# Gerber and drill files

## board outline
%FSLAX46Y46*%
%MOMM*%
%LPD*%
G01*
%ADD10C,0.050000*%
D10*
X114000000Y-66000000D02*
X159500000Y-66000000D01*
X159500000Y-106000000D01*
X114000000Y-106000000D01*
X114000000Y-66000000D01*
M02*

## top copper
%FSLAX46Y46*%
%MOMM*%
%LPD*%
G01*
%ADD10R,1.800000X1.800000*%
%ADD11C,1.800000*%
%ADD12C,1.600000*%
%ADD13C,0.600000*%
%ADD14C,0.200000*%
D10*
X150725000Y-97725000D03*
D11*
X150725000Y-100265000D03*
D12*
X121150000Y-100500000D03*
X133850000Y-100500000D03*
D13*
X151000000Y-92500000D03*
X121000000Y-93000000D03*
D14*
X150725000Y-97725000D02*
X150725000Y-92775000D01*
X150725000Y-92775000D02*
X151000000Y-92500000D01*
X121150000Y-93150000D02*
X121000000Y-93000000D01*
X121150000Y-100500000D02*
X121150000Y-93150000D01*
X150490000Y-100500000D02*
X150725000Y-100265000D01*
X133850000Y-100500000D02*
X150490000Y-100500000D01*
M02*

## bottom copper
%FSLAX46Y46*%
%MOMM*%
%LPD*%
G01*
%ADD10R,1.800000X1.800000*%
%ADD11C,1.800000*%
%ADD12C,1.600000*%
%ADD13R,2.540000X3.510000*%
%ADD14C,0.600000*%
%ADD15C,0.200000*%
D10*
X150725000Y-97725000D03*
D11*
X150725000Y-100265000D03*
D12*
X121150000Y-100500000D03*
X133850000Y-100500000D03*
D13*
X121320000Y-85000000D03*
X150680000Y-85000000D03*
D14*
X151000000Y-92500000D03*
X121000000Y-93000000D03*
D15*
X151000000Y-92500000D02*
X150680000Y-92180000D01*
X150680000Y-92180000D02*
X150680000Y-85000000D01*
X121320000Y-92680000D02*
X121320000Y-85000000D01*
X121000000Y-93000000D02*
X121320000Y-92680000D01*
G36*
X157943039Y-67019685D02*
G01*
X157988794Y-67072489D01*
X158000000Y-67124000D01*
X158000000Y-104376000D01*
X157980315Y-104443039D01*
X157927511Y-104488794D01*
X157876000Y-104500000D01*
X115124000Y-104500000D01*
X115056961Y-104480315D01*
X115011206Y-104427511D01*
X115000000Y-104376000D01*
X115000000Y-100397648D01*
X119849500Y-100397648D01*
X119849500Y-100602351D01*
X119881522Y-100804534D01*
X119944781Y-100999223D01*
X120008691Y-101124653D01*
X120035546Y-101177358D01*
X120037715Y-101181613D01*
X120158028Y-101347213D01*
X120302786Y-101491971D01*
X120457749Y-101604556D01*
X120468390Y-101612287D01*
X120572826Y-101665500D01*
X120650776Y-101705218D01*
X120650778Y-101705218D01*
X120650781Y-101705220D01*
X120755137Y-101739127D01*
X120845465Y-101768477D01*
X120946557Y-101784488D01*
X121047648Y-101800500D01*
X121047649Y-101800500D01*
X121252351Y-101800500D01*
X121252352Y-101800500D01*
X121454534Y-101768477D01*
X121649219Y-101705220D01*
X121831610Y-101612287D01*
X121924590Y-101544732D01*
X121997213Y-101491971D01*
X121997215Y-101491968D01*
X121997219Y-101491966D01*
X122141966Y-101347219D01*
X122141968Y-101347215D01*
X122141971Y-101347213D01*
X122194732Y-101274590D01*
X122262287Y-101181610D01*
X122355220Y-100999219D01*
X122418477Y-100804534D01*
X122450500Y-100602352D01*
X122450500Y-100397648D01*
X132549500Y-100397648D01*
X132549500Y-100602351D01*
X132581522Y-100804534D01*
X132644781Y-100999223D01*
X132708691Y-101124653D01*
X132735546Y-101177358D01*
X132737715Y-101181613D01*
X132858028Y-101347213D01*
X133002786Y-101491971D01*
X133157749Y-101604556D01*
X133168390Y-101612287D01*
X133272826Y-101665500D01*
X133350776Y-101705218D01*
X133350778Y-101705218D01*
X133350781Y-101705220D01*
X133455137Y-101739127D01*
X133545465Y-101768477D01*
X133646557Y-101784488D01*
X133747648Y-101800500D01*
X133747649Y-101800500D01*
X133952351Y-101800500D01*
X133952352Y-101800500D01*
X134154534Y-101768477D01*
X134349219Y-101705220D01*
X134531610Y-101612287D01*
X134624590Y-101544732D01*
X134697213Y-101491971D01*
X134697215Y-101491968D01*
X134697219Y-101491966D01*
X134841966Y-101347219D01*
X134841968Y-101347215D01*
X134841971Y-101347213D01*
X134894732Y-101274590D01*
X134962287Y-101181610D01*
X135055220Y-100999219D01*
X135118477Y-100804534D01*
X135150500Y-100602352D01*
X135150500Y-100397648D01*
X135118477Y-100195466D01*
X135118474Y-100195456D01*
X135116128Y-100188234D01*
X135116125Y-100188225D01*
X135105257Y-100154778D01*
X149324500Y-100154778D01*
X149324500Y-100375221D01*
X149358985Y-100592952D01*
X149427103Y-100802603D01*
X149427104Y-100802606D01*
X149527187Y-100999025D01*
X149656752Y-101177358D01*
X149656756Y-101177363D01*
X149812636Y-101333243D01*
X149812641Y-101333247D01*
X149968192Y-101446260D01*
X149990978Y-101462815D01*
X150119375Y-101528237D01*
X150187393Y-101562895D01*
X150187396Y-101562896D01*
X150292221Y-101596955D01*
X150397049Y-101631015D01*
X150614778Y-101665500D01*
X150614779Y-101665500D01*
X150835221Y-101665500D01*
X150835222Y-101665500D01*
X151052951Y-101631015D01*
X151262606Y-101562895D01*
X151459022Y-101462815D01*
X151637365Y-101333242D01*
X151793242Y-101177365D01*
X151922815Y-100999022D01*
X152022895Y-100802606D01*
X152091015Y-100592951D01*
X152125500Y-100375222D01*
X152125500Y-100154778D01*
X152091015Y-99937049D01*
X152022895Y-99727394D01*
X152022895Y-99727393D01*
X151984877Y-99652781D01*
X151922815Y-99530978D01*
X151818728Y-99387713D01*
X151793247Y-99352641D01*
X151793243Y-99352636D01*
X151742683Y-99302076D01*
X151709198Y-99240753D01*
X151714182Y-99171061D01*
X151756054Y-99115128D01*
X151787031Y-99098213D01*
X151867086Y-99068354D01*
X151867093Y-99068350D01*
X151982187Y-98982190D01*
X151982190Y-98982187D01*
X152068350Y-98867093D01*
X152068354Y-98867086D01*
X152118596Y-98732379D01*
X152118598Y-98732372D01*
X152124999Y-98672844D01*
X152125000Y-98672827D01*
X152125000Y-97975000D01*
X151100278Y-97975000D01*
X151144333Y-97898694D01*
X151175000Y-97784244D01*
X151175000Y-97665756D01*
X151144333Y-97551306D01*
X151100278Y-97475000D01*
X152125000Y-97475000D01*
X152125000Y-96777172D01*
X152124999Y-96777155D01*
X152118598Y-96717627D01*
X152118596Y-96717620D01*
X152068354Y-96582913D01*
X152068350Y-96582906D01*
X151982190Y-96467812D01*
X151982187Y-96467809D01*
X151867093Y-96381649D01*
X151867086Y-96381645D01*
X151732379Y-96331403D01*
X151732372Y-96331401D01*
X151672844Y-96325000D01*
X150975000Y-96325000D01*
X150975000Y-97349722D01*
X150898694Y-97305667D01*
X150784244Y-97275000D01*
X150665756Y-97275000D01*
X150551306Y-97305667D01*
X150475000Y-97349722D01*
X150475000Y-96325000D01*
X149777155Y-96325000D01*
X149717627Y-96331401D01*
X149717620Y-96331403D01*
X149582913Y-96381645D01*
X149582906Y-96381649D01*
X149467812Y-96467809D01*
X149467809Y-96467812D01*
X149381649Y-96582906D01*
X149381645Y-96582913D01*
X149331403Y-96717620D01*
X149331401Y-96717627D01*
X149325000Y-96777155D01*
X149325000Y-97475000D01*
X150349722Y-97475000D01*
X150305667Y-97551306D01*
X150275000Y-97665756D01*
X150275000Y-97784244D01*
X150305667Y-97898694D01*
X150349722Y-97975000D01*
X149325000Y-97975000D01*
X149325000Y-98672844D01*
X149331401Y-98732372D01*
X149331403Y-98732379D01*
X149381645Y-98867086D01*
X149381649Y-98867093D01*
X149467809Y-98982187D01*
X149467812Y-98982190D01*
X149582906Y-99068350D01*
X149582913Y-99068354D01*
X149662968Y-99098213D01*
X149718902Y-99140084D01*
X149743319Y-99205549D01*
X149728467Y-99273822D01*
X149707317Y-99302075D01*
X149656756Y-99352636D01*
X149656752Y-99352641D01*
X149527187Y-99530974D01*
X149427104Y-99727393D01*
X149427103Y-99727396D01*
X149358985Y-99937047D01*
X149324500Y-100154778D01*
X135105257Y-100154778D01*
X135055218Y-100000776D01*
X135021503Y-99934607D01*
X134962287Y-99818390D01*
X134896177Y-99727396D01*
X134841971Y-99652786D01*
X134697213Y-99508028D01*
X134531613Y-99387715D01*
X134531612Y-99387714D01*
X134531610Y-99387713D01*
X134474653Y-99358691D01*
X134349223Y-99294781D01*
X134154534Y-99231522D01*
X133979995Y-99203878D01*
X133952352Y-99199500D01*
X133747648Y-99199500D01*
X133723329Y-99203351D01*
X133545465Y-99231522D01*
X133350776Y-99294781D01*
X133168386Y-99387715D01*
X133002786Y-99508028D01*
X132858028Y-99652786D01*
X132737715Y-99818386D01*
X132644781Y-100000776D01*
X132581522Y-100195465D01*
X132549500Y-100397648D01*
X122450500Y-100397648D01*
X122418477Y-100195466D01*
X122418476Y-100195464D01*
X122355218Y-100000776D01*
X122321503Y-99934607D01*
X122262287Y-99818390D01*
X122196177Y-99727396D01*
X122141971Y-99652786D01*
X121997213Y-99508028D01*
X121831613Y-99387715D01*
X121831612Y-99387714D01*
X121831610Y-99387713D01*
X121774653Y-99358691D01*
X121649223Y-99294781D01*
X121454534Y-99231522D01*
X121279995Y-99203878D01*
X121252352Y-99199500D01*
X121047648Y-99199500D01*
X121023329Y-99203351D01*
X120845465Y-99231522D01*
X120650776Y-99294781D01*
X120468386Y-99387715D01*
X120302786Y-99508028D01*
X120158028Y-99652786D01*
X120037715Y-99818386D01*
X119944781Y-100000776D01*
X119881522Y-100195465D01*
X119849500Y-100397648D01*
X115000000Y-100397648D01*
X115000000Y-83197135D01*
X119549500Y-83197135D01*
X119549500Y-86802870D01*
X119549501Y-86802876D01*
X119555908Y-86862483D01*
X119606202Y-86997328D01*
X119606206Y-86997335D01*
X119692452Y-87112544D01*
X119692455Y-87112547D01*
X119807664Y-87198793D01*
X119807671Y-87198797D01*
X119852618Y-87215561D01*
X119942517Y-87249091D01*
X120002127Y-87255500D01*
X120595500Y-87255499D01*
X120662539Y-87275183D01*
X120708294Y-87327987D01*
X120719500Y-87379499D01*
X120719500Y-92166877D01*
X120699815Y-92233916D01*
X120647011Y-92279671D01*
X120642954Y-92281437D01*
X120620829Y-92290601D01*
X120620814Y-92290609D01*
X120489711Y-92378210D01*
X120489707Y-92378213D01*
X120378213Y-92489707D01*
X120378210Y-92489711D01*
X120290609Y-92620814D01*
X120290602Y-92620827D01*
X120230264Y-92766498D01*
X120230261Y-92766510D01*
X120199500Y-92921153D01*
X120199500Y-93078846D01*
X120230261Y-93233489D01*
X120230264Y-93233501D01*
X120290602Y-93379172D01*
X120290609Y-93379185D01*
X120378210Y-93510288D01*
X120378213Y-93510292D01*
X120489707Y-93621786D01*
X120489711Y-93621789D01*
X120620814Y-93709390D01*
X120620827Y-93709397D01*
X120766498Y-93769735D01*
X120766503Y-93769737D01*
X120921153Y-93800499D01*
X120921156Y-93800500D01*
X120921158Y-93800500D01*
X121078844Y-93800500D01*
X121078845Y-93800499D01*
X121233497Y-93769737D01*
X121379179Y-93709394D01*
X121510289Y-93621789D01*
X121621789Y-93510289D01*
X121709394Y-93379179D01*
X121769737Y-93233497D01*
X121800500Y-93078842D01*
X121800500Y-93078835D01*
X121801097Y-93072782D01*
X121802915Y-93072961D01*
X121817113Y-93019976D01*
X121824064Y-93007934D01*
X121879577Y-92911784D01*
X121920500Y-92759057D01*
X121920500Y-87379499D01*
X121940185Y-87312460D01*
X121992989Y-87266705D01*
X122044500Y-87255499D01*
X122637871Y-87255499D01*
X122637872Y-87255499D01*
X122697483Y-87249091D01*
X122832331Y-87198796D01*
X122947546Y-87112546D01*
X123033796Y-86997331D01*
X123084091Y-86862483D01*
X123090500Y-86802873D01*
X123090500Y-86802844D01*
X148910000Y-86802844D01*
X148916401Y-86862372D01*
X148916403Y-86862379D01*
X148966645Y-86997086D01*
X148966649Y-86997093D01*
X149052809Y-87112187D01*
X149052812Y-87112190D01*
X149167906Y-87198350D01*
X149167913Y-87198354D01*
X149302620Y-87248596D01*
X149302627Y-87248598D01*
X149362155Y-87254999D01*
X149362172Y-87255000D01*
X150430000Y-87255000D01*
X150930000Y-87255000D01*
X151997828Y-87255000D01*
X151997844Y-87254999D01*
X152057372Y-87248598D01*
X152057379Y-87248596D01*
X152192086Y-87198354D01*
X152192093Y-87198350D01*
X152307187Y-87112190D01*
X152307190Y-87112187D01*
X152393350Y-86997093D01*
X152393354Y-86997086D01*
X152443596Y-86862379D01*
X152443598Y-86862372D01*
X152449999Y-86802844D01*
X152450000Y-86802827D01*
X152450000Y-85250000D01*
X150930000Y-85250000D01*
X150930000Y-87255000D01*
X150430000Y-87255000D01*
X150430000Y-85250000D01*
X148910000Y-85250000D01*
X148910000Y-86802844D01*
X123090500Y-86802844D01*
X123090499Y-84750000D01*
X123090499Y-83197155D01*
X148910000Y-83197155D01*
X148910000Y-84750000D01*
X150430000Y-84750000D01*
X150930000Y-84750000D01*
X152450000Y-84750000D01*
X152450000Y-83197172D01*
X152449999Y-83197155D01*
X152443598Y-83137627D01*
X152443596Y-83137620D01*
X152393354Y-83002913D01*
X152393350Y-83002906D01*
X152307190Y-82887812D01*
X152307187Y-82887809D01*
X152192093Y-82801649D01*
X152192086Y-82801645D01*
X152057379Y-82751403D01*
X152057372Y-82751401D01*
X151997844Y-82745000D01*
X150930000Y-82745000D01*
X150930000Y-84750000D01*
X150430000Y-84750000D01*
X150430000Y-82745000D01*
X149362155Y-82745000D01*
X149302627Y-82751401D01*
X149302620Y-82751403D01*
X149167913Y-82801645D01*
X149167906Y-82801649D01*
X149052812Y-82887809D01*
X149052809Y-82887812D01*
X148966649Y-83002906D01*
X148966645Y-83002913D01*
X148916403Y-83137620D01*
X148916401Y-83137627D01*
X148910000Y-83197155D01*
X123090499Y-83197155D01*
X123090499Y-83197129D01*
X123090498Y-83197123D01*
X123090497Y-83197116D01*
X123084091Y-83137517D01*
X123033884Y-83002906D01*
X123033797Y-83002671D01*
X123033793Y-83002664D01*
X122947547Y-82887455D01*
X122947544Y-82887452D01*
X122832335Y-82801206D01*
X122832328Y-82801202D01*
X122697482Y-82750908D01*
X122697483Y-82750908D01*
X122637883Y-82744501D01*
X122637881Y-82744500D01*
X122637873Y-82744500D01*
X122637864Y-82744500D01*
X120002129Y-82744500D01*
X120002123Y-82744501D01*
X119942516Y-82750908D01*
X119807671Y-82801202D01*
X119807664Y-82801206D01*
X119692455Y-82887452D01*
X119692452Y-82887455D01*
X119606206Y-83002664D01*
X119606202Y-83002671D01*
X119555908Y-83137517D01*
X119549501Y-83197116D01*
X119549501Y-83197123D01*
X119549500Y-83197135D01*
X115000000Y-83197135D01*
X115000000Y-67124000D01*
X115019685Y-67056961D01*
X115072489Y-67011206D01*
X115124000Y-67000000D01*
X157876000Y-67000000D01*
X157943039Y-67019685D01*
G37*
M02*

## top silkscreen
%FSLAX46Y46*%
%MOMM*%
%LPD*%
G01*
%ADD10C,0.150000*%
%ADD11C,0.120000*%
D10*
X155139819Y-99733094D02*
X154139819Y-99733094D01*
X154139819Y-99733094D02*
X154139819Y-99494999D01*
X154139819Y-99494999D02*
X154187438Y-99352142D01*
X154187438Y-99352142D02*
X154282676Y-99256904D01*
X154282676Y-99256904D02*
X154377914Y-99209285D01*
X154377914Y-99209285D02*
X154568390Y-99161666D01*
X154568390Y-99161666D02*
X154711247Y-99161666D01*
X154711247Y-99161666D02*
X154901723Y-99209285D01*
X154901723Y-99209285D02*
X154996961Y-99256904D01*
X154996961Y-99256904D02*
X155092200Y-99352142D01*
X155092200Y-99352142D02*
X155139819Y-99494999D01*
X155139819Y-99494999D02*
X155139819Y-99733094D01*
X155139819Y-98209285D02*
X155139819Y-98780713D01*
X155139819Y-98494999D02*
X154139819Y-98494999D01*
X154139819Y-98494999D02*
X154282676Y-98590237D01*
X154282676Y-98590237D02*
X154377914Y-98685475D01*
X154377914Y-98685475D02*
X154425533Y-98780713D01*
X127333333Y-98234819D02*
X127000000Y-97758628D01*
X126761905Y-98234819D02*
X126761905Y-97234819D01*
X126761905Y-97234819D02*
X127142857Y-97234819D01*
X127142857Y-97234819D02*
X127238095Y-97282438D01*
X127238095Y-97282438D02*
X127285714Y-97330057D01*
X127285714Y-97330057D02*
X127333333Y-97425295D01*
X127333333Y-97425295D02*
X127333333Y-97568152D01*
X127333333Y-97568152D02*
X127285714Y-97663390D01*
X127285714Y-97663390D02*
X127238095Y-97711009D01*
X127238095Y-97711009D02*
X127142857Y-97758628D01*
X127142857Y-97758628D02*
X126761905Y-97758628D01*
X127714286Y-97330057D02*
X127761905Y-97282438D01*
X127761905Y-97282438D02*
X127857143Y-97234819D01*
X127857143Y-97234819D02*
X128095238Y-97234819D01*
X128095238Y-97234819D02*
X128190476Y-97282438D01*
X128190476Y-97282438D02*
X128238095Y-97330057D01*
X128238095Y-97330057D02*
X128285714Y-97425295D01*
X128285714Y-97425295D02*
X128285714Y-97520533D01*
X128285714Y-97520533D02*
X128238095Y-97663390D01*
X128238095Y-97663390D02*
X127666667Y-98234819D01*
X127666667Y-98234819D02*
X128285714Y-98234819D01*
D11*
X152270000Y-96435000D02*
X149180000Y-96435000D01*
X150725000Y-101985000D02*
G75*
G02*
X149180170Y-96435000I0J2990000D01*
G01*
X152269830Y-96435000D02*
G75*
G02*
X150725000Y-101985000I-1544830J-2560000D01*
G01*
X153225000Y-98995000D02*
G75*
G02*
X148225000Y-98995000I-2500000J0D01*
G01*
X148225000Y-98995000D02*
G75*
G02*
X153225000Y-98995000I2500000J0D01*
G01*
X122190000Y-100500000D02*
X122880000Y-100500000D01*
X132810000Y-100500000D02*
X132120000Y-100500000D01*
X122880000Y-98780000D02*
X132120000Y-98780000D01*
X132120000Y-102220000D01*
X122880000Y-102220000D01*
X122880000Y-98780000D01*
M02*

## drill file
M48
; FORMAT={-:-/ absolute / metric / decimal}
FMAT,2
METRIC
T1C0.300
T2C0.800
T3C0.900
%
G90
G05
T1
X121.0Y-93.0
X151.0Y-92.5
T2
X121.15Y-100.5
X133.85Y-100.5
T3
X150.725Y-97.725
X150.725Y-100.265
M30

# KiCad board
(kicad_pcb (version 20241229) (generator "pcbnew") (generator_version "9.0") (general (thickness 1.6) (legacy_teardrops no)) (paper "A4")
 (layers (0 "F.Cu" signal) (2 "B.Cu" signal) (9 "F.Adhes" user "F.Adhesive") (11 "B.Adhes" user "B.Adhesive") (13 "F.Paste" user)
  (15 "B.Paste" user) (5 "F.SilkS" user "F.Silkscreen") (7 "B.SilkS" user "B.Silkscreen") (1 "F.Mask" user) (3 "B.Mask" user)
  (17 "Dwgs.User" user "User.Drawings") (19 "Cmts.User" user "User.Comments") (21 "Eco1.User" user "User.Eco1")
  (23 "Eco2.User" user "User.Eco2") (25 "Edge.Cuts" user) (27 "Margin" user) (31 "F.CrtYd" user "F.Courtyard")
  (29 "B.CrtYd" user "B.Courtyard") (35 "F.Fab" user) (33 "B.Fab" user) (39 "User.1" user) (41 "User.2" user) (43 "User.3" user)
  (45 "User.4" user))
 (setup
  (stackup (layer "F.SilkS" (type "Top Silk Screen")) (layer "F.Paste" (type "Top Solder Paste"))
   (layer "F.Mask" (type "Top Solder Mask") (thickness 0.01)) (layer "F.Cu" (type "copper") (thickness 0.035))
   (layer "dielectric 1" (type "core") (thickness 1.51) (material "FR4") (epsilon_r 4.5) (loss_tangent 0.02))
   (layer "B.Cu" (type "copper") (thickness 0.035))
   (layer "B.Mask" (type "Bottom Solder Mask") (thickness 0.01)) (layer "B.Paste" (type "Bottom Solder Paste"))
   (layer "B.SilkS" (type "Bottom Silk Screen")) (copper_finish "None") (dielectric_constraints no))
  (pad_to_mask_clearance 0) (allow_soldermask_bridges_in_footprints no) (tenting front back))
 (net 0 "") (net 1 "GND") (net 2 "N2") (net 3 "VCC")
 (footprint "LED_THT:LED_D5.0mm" (layer "F.Cu") (at 150.725 97.725 -90)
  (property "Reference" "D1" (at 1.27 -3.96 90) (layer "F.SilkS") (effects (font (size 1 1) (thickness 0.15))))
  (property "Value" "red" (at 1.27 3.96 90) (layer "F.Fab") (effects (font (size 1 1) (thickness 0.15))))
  (fp_line (start -1.29 -1.545) (end -1.29 1.545) (stroke (width 0.12) (type solid)) (layer "F.SilkS"))
  (fp_arc (start 4.26 0) (mid 2.071779 2.880495) (end -1.29 1.54483) (stroke (width 0.12) (type solid)) (layer "F.SilkS"))
  (fp_arc (start -1.29 -1.54483) (mid 2.071779 -2.880495) (end 4.26 0) (stroke (width 0.12) (type solid)) (layer "F.SilkS"))
  (fp_circle (center 1.27 0) (end 3.77 0) (stroke (width 0.12) (type solid)) (fill no) (layer "F.SilkS"))
  (pad "1" thru_hole rect (at 0 0 270) (size 1.8 1.8) (drill 0.9) (layers "*.Cu" "*.Mask") (remove_unused_layers no) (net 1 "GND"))
  (pad "2" thru_hole circle (at 2.54 0 270) (size 1.8 1.8) (drill 0.9) (layers "*.Cu" "*.Mask") (remove_unused_layers no) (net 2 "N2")))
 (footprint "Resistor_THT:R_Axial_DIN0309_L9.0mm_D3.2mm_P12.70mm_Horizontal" (layer "F.Cu") (at 121.15 100.5)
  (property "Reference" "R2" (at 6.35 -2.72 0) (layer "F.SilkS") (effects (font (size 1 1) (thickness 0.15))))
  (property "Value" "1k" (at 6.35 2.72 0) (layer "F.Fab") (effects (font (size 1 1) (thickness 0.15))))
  (fp_line (start 1.04 0) (end 1.73 0) (stroke (width 0.12) (type solid)) (layer "F.SilkS"))
  (fp_line (start 11.66 0) (end 10.97 0) (stroke (width 0.12) (type solid)) (layer "F.SilkS"))
  (fp_rect (start 1.73 -1.72) (end 10.97 1.72) (stroke (width 0.12) (type solid)) (fill no) (layer "F.SilkS"))
  (pad "1" thru_hole circle (at 0 0) (size 1.6 1.6) (drill 0.8) (layers "*.Cu" "*.Mask") (remove_unused_layers no) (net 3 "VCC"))
  (pad "2" thru_hole circle (at 12.7 0) (size 1.6 1.6) (drill 0.8) (layers "*.Cu" "*.Mask") (remove_unused_layers no) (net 2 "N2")))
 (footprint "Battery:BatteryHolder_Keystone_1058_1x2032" (layer "B.Cu") (at 136 85)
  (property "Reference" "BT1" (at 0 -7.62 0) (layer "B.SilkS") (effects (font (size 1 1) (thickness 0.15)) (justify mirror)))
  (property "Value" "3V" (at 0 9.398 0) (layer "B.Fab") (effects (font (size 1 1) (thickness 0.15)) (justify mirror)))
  (pad "1" smd rect (at -14.68 0) (size 2.54 3.51) (layers "B.Cu" "B.Mask" "B.Paste") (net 3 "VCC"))
  (pad "2" smd rect (at 14.68 0) (size 2.54 3.51) (layers "B.Cu" "B.Mask" "B.Paste") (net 1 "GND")))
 (gr_rect (start 114 66) (end 159.5 106) (stroke (width 0.05) (type default)) (fill no) (layer "Edge.Cuts"))
 (segment (start 150.725 97.725) (end 150.725 92.775) (width 0.2) (layer "F.Cu") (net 1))
 (segment (start 150.725 92.775) (end 151 92.5) (width 0.2) (layer "F.Cu") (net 1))
 (via (at 151 92.5) (size 0.6) (drill 0.3) (layers "F.Cu" "B.Cu") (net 1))
 (segment (start 151 92.5) (end 150.68 92.18) (width 0.2) (layer "B.Cu") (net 1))
 (segment (start 150.68 92.18) (end 150.68 85) (width 0.2) (layer "B.Cu") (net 1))
 (segment (start 121.15 93.15) (end 121 93) (width 0.2) (layer "F.Cu") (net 3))
 (segment (start 121.15 100.5) (end 121.15 93.15) (width 0.2) (layer "F.Cu") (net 3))
 (via (at 121 93) (size 0.6) (drill 0.3) (layers "F.Cu" "B.Cu") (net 3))
 (segment (start 121.32 92.68) (end 121.32 85) (width 0.2) (layer "B.Cu") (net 3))
 (segment (start 121 93) (end 121.32 92.68) (width 0.2) (layer "B.Cu") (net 3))
 (segment (start 150.49 100.5) (end 150.725 100.265) (width 0.2) (layer "F.Cu") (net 2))
 (segment (start 133.85 100.5) (end 150.49 100.5) (width 0.2) (layer "F.Cu") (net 2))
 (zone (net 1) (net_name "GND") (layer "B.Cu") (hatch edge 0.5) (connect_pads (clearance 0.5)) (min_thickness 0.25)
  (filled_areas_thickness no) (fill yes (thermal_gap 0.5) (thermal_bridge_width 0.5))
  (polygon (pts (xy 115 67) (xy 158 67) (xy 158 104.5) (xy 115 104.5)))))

